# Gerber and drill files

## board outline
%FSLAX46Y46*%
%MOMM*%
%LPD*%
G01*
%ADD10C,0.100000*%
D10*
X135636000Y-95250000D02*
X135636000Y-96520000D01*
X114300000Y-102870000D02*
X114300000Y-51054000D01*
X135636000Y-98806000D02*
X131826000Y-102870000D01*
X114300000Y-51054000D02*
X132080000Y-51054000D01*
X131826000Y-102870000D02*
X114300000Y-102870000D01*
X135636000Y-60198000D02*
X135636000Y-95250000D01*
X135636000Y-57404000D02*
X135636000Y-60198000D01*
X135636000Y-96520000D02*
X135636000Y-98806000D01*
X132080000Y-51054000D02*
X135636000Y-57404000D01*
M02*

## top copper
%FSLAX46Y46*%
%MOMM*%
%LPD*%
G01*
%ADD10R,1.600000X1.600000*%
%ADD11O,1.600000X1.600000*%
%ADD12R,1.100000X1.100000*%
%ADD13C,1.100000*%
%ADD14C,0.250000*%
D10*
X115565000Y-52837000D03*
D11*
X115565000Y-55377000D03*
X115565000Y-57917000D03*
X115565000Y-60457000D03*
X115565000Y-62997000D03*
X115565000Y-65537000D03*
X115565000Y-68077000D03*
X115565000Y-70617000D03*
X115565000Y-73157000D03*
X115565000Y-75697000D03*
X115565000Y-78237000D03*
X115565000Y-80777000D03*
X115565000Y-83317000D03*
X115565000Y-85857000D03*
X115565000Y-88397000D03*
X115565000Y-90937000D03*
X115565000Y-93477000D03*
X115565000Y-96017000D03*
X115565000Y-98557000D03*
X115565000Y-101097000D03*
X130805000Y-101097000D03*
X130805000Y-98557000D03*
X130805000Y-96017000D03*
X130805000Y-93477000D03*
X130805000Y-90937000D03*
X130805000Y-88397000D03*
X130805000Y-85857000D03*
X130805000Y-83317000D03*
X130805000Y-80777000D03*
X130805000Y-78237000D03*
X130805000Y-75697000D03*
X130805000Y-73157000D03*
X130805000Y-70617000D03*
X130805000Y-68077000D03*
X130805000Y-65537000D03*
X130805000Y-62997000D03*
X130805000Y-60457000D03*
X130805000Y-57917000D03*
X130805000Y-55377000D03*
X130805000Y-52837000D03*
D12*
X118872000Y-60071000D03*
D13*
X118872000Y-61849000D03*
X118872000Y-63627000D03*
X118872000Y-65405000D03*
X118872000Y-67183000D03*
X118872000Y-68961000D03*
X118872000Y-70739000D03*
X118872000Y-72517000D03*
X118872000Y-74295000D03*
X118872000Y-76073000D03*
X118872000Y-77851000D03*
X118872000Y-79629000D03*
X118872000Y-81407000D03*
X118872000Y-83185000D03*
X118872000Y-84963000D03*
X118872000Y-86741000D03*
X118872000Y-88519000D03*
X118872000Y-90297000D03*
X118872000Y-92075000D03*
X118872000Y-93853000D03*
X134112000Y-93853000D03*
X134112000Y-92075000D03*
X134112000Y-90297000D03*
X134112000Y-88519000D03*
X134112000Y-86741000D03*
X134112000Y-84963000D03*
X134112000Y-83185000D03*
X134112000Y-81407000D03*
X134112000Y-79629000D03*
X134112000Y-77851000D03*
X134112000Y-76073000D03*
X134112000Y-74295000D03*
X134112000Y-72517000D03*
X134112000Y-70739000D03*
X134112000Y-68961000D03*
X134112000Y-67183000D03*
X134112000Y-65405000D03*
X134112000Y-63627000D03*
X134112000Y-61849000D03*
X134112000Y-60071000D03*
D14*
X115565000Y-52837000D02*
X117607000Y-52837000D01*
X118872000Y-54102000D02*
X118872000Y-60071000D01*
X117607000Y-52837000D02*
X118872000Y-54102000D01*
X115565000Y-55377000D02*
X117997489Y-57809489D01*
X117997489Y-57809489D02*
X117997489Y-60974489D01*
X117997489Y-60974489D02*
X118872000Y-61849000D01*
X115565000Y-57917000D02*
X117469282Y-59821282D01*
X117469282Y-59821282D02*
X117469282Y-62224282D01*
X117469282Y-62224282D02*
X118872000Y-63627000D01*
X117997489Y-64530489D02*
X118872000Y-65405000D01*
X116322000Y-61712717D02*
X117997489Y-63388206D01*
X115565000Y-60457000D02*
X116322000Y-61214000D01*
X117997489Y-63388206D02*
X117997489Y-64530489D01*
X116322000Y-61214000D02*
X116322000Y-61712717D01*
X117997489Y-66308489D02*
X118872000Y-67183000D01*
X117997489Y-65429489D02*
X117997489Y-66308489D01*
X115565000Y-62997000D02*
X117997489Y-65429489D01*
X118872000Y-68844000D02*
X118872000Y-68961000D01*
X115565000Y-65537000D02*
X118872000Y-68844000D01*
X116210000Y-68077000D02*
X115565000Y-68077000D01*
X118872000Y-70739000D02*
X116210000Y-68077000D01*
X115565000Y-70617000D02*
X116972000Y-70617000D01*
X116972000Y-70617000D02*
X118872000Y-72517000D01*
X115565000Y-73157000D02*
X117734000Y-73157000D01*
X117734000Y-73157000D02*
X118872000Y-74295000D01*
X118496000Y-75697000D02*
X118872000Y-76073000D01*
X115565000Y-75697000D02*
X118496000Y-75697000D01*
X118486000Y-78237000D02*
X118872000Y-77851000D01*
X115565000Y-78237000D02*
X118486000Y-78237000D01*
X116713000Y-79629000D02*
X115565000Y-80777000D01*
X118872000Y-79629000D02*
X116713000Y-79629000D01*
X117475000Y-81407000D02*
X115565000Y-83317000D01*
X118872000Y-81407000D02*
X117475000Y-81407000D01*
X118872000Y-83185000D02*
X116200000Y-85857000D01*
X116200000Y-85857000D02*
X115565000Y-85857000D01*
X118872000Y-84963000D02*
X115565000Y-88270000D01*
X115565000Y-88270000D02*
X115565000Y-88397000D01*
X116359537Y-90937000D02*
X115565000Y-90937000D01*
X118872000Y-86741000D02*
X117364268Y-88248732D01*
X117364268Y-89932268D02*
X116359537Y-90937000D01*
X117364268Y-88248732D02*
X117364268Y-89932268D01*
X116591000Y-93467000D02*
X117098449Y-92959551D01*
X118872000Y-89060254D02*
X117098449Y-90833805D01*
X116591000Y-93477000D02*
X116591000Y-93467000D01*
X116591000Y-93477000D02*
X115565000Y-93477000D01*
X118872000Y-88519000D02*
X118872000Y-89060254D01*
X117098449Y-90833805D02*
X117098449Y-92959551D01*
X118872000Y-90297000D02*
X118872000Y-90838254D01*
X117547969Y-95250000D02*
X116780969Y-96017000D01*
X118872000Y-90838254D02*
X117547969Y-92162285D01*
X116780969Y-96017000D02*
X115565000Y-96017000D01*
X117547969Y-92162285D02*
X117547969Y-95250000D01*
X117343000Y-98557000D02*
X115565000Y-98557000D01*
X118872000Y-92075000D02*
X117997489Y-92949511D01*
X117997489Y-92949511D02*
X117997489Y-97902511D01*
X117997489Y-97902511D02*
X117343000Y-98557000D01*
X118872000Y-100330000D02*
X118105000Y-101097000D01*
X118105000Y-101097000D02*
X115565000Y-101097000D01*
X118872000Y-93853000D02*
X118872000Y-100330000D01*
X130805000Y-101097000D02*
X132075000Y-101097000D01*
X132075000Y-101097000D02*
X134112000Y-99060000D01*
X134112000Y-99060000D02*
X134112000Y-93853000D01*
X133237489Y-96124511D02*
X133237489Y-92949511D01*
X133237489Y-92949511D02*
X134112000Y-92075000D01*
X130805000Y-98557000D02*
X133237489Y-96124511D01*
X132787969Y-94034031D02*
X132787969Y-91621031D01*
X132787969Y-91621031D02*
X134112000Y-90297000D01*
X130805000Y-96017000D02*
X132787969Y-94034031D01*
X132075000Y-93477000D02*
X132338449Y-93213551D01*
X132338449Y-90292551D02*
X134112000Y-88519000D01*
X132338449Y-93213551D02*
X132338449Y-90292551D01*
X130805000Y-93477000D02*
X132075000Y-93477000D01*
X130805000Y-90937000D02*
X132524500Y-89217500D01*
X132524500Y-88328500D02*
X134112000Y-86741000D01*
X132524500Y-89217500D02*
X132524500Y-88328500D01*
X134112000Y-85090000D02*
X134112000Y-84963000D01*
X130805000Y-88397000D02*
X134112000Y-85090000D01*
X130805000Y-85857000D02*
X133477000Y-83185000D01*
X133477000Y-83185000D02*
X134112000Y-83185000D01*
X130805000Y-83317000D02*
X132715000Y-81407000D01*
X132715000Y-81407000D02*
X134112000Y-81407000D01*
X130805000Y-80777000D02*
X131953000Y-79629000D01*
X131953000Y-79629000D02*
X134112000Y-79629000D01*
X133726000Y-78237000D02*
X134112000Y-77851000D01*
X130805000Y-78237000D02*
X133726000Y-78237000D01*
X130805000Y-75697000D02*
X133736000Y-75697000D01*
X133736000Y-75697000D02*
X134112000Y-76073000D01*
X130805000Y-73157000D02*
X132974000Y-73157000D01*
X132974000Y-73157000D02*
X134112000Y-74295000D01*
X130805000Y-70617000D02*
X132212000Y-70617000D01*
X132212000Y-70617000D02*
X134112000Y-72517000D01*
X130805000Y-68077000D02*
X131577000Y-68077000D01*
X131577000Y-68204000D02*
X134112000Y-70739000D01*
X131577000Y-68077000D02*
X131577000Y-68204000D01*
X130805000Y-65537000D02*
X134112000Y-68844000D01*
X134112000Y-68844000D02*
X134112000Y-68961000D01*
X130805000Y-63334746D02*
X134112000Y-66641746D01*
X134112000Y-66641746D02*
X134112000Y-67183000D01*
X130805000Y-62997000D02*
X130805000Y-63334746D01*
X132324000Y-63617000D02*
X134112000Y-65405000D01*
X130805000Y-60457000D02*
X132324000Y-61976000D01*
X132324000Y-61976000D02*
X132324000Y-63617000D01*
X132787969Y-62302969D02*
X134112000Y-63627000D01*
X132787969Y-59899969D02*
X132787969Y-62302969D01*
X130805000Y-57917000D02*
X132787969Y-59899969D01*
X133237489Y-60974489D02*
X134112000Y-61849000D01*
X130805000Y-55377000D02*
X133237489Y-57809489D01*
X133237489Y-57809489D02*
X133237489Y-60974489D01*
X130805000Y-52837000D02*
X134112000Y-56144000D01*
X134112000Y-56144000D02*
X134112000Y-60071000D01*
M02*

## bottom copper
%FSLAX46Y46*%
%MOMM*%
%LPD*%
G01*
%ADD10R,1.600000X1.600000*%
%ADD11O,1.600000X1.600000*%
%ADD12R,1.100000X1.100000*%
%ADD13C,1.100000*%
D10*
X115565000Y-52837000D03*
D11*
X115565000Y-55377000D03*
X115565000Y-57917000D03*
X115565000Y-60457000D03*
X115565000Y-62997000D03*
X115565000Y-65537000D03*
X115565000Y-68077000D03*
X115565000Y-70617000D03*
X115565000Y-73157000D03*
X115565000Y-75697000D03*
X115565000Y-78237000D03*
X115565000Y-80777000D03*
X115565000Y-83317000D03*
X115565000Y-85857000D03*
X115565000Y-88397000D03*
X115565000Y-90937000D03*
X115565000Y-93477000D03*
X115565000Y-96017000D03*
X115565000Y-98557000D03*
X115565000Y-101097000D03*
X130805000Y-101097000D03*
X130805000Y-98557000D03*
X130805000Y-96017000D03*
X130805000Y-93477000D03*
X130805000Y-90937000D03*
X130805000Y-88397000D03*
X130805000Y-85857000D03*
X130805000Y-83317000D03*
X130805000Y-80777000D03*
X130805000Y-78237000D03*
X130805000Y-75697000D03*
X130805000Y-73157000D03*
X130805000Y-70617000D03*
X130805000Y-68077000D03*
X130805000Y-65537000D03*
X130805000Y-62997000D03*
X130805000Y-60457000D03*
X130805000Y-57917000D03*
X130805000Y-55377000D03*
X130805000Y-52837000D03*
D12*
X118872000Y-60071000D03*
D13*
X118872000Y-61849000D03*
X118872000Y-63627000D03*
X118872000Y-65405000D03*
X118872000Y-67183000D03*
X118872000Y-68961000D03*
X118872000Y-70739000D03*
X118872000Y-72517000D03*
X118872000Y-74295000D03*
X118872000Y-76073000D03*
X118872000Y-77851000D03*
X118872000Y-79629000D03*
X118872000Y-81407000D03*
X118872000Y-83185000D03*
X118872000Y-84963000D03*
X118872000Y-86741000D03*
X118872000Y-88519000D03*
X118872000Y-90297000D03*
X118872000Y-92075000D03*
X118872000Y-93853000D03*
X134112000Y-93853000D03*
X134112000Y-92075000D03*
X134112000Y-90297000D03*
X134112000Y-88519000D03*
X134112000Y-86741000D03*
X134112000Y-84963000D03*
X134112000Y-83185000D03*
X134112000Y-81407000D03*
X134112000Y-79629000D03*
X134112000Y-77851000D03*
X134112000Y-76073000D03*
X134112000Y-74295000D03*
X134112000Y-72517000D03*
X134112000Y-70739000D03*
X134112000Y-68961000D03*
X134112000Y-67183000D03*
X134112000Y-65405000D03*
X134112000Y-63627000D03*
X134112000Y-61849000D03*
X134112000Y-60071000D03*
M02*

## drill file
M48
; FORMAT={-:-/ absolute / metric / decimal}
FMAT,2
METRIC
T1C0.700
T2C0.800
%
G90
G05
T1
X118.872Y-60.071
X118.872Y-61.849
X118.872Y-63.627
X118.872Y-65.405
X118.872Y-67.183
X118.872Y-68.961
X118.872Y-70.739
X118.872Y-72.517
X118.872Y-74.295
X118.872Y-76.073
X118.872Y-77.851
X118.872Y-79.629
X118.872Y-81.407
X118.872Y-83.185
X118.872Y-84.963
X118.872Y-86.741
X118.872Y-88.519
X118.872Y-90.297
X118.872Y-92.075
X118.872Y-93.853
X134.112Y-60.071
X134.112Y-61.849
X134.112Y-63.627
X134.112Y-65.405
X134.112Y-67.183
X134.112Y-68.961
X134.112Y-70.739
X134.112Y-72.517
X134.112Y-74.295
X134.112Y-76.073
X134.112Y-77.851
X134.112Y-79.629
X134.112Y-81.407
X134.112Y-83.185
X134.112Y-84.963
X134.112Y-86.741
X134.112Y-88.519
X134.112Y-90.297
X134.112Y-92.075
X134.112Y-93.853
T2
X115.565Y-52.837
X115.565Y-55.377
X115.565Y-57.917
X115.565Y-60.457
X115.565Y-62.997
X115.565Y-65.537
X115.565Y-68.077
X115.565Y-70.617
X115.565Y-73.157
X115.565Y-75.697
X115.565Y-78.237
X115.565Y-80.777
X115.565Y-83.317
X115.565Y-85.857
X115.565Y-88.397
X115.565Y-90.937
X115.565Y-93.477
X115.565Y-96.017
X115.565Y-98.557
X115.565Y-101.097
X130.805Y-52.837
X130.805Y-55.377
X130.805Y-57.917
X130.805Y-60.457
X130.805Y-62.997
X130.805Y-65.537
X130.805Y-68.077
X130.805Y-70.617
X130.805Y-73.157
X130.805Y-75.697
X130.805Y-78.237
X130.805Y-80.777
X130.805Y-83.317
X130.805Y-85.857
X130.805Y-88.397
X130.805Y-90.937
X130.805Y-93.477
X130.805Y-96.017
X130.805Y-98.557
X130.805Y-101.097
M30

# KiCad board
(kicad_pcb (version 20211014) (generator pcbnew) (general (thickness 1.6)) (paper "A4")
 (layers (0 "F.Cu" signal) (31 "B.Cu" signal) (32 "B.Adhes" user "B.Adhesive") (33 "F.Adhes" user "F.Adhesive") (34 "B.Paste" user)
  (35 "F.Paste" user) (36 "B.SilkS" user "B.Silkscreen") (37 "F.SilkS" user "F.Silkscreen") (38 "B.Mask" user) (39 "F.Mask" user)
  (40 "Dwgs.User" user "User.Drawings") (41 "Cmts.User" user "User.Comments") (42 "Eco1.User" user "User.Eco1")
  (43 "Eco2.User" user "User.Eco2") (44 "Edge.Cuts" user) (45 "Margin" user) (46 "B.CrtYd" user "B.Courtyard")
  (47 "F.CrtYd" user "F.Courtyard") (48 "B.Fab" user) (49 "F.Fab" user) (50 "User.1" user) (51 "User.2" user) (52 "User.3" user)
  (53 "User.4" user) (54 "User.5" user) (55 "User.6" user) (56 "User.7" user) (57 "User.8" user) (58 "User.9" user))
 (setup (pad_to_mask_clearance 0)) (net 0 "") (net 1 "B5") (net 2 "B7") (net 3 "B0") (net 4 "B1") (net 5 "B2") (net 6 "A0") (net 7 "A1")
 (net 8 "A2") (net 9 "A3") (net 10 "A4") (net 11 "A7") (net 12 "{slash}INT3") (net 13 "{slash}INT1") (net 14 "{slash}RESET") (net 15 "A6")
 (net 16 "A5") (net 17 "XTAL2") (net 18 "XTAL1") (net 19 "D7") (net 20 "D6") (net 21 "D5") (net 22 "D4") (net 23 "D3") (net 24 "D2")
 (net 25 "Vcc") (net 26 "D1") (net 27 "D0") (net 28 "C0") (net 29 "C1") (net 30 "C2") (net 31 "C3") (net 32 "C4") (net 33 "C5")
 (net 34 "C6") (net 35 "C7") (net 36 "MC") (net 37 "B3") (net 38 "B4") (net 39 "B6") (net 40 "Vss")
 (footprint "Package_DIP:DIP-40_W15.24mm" (layer "F.Cu") (at 115.565 52.837)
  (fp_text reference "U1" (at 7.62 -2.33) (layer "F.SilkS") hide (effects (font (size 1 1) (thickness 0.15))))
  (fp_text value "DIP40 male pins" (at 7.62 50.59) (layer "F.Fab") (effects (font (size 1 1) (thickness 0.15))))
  (pad "1" thru_hole rect locked (at 0 0) (size 1.6 1.6) (drill 0.8) (layers *.Cu *.Mask) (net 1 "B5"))
  (pad "2" thru_hole oval locked (at 0 2.54) (size 1.6 1.6) (drill 0.8) (layers *.Cu *.Mask) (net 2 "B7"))
  (pad "3" thru_hole oval locked (at 0 5.08) (size 1.6 1.6) (drill 0.8) (layers *.Cu *.Mask) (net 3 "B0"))
  (pad "4" thru_hole oval locked (at 0 7.62) (size 1.6 1.6) (drill 0.8) (layers *.Cu *.Mask) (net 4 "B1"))
  (pad "5" thru_hole oval locked (at 0 10.16) (size 1.6 1.6) (drill 0.8) (layers *.Cu *.Mask) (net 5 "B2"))
  (pad "6" thru_hole oval locked (at 0 12.7) (size 1.6 1.6) (drill 0.8) (layers *.Cu *.Mask) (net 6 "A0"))
  (pad "7" thru_hole oval locked (at 0 15.24) (size 1.6 1.6) (drill 0.8) (layers *.Cu *.Mask) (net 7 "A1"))
  (pad "8" thru_hole oval locked (at 0 17.78) (size 1.6 1.6) (drill 0.8) (layers *.Cu *.Mask) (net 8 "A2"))
  (pad "9" thru_hole oval locked (at 0 20.32) (size 1.6 1.6) (drill 0.8) (layers *.Cu *.Mask) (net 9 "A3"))
  (pad "10" thru_hole oval locked (at 0 22.86) (size 1.6 1.6) (drill 0.8) (layers *.Cu *.Mask) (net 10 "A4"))
  (pad "11" thru_hole oval locked (at 0 25.4) (size 1.6 1.6) (drill 0.8) (layers *.Cu *.Mask) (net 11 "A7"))
  (pad "12" thru_hole oval locked (at 0 27.94) (size 1.6 1.6) (drill 0.8) (layers *.Cu *.Mask) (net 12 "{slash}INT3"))
  (pad "13" thru_hole oval locked (at 0 30.48) (size 1.6 1.6) (drill 0.8) (layers *.Cu *.Mask) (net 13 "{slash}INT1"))
  (pad "14" thru_hole oval locked (at 0 33.02) (size 1.6 1.6) (drill 0.8) (layers *.Cu *.Mask) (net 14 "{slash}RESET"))
  (pad "15" thru_hole oval locked (at 0 35.56) (size 1.6 1.6) (drill 0.8) (layers *.Cu *.Mask) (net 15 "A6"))
  (pad "16" thru_hole oval locked (at 0 38.1) (size 1.6 1.6) (drill 0.8) (layers *.Cu *.Mask) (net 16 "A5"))
  (pad "17" thru_hole oval locked (at 0 40.64) (size 1.6 1.6) (drill 0.8) (layers *.Cu *.Mask) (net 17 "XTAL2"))
  (pad "18" thru_hole oval locked (at 0 43.18) (size 1.6 1.6) (drill 0.8) (layers *.Cu *.Mask) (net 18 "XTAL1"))
  (pad "19" thru_hole oval locked (at 0 45.72) (size 1.6 1.6) (drill 0.8) (layers *.Cu *.Mask) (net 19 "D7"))
  (pad "20" thru_hole oval locked (at 0 48.26) (size 1.6 1.6) (drill 0.8) (layers *.Cu *.Mask) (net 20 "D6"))
  (pad "21" thru_hole oval locked (at 15.24 48.26) (size 1.6 1.6) (drill 0.8) (layers *.Cu *.Mask) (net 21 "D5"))
  (pad "22" thru_hole oval locked (at 15.24 45.72) (size 1.6 1.6) (drill 0.8) (layers *.Cu *.Mask) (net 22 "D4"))
  (pad "23" thru_hole oval locked (at 15.24 43.18) (size 1.6 1.6) (drill 0.8) (layers *.Cu *.Mask) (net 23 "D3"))
  (pad "24" thru_hole oval locked (at 15.24 40.64) (size 1.6 1.6) (drill 0.8) (layers *.Cu *.Mask) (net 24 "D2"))
  (pad "25" thru_hole oval locked (at 15.24 38.1) (size 1.6 1.6) (drill 0.8) (layers *.Cu *.Mask) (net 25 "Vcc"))
  (pad "26" thru_hole oval locked (at 15.24 35.56) (size 1.6 1.6) (drill 0.8) (layers *.Cu *.Mask) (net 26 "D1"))
  (pad "27" thru_hole oval locked (at 15.24 33.02) (size 1.6 1.6) (drill 0.8) (layers *.Cu *.Mask) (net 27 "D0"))
  (pad "28" thru_hole oval locked (at 15.24 30.48) (size 1.6 1.6) (drill 0.8) (layers *.Cu *.Mask) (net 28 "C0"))
  (pad "29" thru_hole oval locked (at 15.24 27.94) (size 1.6 1.6) (drill 0.8) (layers *.Cu *.Mask) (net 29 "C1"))
  (pad "30" thru_hole oval locked (at 15.24 25.4) (size 1.6 1.6) (drill 0.8) (layers *.Cu *.Mask) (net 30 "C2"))
  (pad "31" thru_hole oval locked (at 15.24 22.86) (size 1.6 1.6) (drill 0.8) (layers *.Cu *.Mask) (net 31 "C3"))
  (pad "32" thru_hole oval locked (at 15.24 20.32) (size 1.6 1.6) (drill 0.8) (layers *.Cu *.Mask) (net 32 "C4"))
  (pad "33" thru_hole oval locked (at 15.24 17.78) (size 1.6 1.6) (drill 0.8) (layers *.Cu *.Mask) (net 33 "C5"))
  (pad "34" thru_hole oval locked (at 15.24 15.24) (size 1.6 1.6) (drill 0.8) (layers *.Cu *.Mask) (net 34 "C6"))
  (pad "35" thru_hole oval locked (at 15.24 12.7) (size 1.6 1.6) (drill 0.8) (layers *.Cu *.Mask) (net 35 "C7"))
  (pad "36" thru_hole oval locked (at 15.24 10.16) (size 1.6 1.6) (drill 0.8) (layers *.Cu *.Mask) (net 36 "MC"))
  (pad "37" thru_hole oval locked (at 15.24 7.62) (size 1.6 1.6) (drill 0.8) (layers *.Cu *.Mask) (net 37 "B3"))
  (pad "38" thru_hole oval locked (at 15.24 5.08) (size 1.6 1.6) (drill 0.8) (layers *.Cu *.Mask) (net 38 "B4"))
  (pad "39" thru_hole oval locked (at 15.24 2.54) (size 1.6 1.6) (drill 0.8) (layers *.Cu *.Mask) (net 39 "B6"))
  (pad "40" thru_hole oval locked (at 15.24 0) (size 1.6 1.6) (drill 0.8) (layers *.Cu *.Mask) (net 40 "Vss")))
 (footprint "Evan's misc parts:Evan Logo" (layer "F.Cu") (at 123.444 99.568)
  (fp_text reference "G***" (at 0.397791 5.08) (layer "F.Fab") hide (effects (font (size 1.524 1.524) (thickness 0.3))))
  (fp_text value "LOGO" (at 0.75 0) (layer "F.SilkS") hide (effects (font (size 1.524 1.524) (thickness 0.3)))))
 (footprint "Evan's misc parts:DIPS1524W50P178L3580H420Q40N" (layer "F.Cu") (at 118.872 60.071)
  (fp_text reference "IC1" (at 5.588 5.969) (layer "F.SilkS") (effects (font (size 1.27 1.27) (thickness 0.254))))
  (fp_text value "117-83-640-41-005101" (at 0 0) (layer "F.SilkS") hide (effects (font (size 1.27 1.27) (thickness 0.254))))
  (pad "1" thru_hole rect (at 0 0) (size 1.1 1.1) (drill 0.7) (layers *.Cu *.Mask) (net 1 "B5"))
  (pad "2" thru_hole circle (at 0 1.778) (size 1.1 1.1) (drill 0.7) (layers *.Cu *.Mask) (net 2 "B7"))
  (pad "3" thru_hole circle (at 0 3.556) (size 1.1 1.1) (drill 0.7) (layers *.Cu *.Mask) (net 3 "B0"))
  (pad "4" thru_hole circle (at 0 5.334) (size 1.1 1.1) (drill 0.7) (layers *.Cu *.Mask) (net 4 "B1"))
  (pad "5" thru_hole circle (at 0 7.112) (size 1.1 1.1) (drill 0.7) (layers *.Cu *.Mask) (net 5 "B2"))
  (pad "6" thru_hole circle (at 0 8.89) (size 1.1 1.1) (drill 0.7) (layers *.Cu *.Mask) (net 6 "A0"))
  (pad "7" thru_hole circle (at 0 10.668) (size 1.1 1.1) (drill 0.7) (layers *.Cu *.Mask) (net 7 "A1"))
  (pad "8" thru_hole circle (at 0 12.446) (size 1.1 1.1) (drill 0.7) (layers *.Cu *.Mask) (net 8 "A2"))
  (pad "9" thru_hole circle (at 0 14.224) (size 1.1 1.1) (drill 0.7) (layers *.Cu *.Mask) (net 9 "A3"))
  (pad "10" thru_hole circle (at 0 16.002) (size 1.1 1.1) (drill 0.7) (layers *.Cu *.Mask) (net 10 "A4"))
  (pad "11" thru_hole circle (at 0 17.78) (size 1.1 1.1) (drill 0.7) (layers *.Cu *.Mask) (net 11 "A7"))
  (pad "12" thru_hole circle (at 0 19.558) (size 1.1 1.1) (drill 0.7) (layers *.Cu *.Mask) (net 12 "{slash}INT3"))
  (pad "13" thru_hole circle (at 0 21.336) (size 1.1 1.1) (drill 0.7) (layers *.Cu *.Mask) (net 13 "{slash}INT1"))
  (pad "14" thru_hole circle (at 0 23.114) (size 1.1 1.1) (drill 0.7) (layers *.Cu *.Mask) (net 14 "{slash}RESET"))
  (pad "15" thru_hole circle (at 0 24.892) (size 1.1 1.1) (drill 0.7) (layers *.Cu *.Mask) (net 15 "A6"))
  (pad "16" thru_hole circle (at 0 26.67) (size 1.1 1.1) (drill 0.7) (layers *.Cu *.Mask) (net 16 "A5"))
  (pad "17" thru_hole circle (at 0 28.448) (size 1.1 1.1) (drill 0.7) (layers *.Cu *.Mask) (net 17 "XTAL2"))
  (pad "18" thru_hole circle (at 0 30.226) (size 1.1 1.1) (drill 0.7) (layers *.Cu *.Mask) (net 18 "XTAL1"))
  (pad "19" thru_hole circle (at 0 32.004) (size 1.1 1.1) (drill 0.7) (layers *.Cu *.Mask) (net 19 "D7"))
  (pad "20" thru_hole circle (at 0 33.782) (size 1.1 1.1) (drill 0.7) (layers *.Cu *.Mask) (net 20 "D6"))
  (pad "21" thru_hole circle (at 15.24 33.782) (size 1.1 1.1) (drill 0.7) (layers *.Cu *.Mask) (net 21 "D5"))
  (pad "22" thru_hole circle (at 15.24 32.004) (size 1.1 1.1) (drill 0.7) (layers *.Cu *.Mask) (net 22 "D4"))
  (pad "23" thru_hole circle (at 15.24 30.226) (size 1.1 1.1) (drill 0.7) (layers *.Cu *.Mask) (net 23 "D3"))
  (pad "24" thru_hole circle (at 15.24 28.448) (size 1.1 1.1) (drill 0.7) (layers *.Cu *.Mask) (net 24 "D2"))
  (pad "25" thru_hole circle (at 15.24 26.67) (size 1.1 1.1) (drill 0.7) (layers *.Cu *.Mask) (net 25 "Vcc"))
  (pad "26" thru_hole circle (at 15.24 24.892) (size 1.1 1.1) (drill 0.7) (layers *.Cu *.Mask) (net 26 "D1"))
  (pad "27" thru_hole circle (at 15.24 23.114) (size 1.1 1.1) (drill 0.7) (layers *.Cu *.Mask) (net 27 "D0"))
  (pad "28" thru_hole circle (at 15.24 21.336) (size 1.1 1.1) (drill 0.7) (layers *.Cu *.Mask) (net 28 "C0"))
  (pad "29" thru_hole circle (at 15.24 19.558) (size 1.1 1.1) (drill 0.7) (layers *.Cu *.Mask) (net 29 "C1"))
  (pad "30" thru_hole circle (at 15.24 17.78) (size 1.1 1.1) (drill 0.7) (layers *.Cu *.Mask) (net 30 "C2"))
  (pad "31" thru_hole circle (at 15.24 16.002) (size 1.1 1.1) (drill 0.7) (layers *.Cu *.Mask) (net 31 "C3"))
  (pad "32" thru_hole circle (at 15.24 14.224) (size 1.1 1.1) (drill 0.7) (layers *.Cu *.Mask) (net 32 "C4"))
  (pad "33" thru_hole circle (at 15.24 12.446) (size 1.1 1.1) (drill 0.7) (layers *.Cu *.Mask) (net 33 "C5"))
  (pad "34" thru_hole circle (at 15.24 10.668) (size 1.1 1.1) (drill 0.7) (layers *.Cu *.Mask) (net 34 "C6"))
  (pad "35" thru_hole circle (at 15.24 8.89) (size 1.1 1.1) (drill 0.7) (layers *.Cu *.Mask) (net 35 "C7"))
  (pad "36" thru_hole circle (at 15.24 7.112) (size 1.1 1.1) (drill 0.7) (layers *.Cu *.Mask) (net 36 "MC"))
  (pad "37" thru_hole circle (at 15.24 5.334) (size 1.1 1.1) (drill 0.7) (layers *.Cu *.Mask) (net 37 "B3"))
  (pad "38" thru_hole circle (at 15.24 3.556) (size 1.1 1.1) (drill 0.7) (layers *.Cu *.Mask) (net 38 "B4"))
  (pad "39" thru_hole circle (at 15.24 1.778) (size 1.1 1.1) (drill 0.7) (layers *.Cu *.Mask) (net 39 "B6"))
  (pad "40" thru_hole circle (at 15.24 0) (size 1.1 1.1) (drill 0.7) (layers *.Cu *.Mask) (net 40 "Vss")))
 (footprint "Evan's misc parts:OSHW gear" (layer "B.Cu") (at 123.444 98.552 180)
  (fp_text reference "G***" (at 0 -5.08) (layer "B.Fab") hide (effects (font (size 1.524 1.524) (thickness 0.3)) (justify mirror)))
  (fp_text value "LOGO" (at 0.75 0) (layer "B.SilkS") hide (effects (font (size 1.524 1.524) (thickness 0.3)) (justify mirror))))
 (gr_line (start 135.636 95.25) (end 135.636 96.52) (layer "Edge.Cuts") (width 0.1))
 (gr_line (start 114.3 102.87) (end 114.3 51.054) (layer "Edge.Cuts") (width 0.1))
 (gr_line (start 135.636 98.806) (end 131.826 102.87) (layer "Edge.Cuts") (width 0.1))
 (gr_line (start 114.3 51.054) (end 132.08 51.054) (layer "Edge.Cuts") (width 0.1))
 (gr_line (start 131.826 102.87) (end 114.3 102.87) (layer "Edge.Cuts") (width 0.1))
 (gr_line (start 135.636 60.198) (end 135.636 95.25) (layer "Edge.Cuts") (width 0.1))
 (gr_line (start 135.636 57.404) (end 135.636 60.198) (layer "Edge.Cuts") (width 0.1))
 (gr_line (start 135.636 96.52) (end 135.636 98.806) (layer "Edge.Cuts") (width 0.1))
 (gr_line (start 132.08 51.054) (end 135.636 57.404) (layer "Edge.Cuts") (width 0.1))
 (segment (start 115.565 52.837) (end 117.607 52.837) (width 0.25) (layer "F.Cu") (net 1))
 (segment (start 118.872 54.102) (end 118.872 60.071) (width 0.25) (layer "F.Cu") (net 1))
 (segment (start 117.607 52.837) (end 118.872 54.102) (width 0.25) (layer "F.Cu") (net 1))
 (segment (start 115.565 55.377) (end 117.997489 57.809489) (width 0.25) (layer "F.Cu") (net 2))
 (segment (start 117.997489 57.809489) (end 117.997489 60.974489) (width 0.25) (layer "F.Cu") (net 2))
 (segment (start 117.997489 60.974489) (end 118.872 61.849) (width 0.25) (layer "F.Cu") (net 2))
 (segment (start 115.565 57.917) (end 117.469282 59.821282) (width 0.25) (layer "F.Cu") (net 3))
 (segment (start 117.469282 59.821282) (end 117.469282 62.224282) (width 0.25) (layer "F.Cu") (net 3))
 (segment (start 117.469282 62.224282) (end 118.872 63.627) (width 0.25) (layer "F.Cu") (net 3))
 (segment (start 117.997489 64.530489) (end 118.872 65.405) (width 0.25) (layer "F.Cu") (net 4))
 (segment (start 116.322 61.712717) (end 117.997489 63.388206) (width 0.25) (layer "F.Cu") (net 4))
 (segment (start 115.565 60.457) (end 116.322 61.214) (width 0.25) (layer "F.Cu") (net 4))
 (segment (start 117.997489 63.388206) (end 117.997489 64.530489) (width 0.25) (layer "F.Cu") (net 4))
 (segment (start 116.322 61.214) (end 116.322 61.712717) (width 0.25) (layer "F.Cu") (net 4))
 (segment (start 117.997489 66.308489) (end 118.872 67.183) (width 0.25) (layer "F.Cu") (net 5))
 (segment (start 117.997489 65.429489) (end 117.997489 66.308489) (width 0.25) (layer "F.Cu") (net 5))
 (segment (start 115.565 62.997) (end 117.997489 65.429489) (width 0.25) (layer "F.Cu") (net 5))
 (segment (start 118.872 68.844) (end 118.872 68.961) (width 0.25) (layer "F.Cu") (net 6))
 (segment (start 115.565 65.537) (end 118.872 68.844) (width 0.25) (layer "F.Cu") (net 6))
 (segment (start 116.21 68.077) (end 115.565 68.077) (width 0.25) (layer "F.Cu") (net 7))
 (segment (start 118.872 70.739) (end 116.21 68.077) (width 0.25) (layer "F.Cu") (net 7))
 (segment (start 115.565 70.617) (end 116.972 70.617) (width 0.25) (layer "F.Cu") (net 8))
 (segment (start 116.972 70.617) (end 118.872 72.517) (width 0.25) (layer "F.Cu") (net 8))
 (segment (start 115.565 73.157) (end 117.734 73.157) (width 0.25) (layer "F.Cu") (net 9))
 (segment (start 117.734 73.157) (end 118.872 74.295) (width 0.25) (layer "F.Cu") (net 9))
 (segment (start 118.496 75.697) (end 118.872 76.073) (width 0.25) (layer "F.Cu") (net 10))
 (segment (start 115.565 75.697) (end 118.496 75.697) (width 0.25) (layer "F.Cu") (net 10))
 (segment (start 118.486 78.237) (end 118.872 77.851) (width 0.25) (layer "F.Cu") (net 11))
 (segment (start 115.565 78.237) (end 118.486 78.237) (width 0.25) (layer "F.Cu") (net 11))
 (segment (start 116.713 79.629) (end 115.565 80.777) (width 0.25) (layer "F.Cu") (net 12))
 (segment (start 118.872 79.629) (end 116.713 79.629) (width 0.25) (layer "F.Cu") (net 12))
 (segment (start 117.475 81.407) (end 115.565 83.317) (width 0.25) (layer "F.Cu") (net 13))
 (segment (start 118.872 81.407) (end 117.475 81.407) (width 0.25) (layer "F.Cu") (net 13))
 (segment (start 118.872 83.185) (end 116.2 85.857) (width 0.25) (layer "F.Cu") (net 14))
 (segment (start 116.2 85.857) (end 115.565 85.857) (width 0.25) (layer "F.Cu") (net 14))
 (segment (start 118.872 84.963) (end 115.565 88.27) (width 0.25) (layer "F.Cu") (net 15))
 (segment (start 115.565 88.27) (end 115.565 88.397) (width 0.25) (layer "F.Cu") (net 15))
 (segment (start 116.359537 90.937) (end 115.565 90.937) (width 0.25) (layer "F.Cu") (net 16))
 (segment (start 118.872 86.741) (end 117.364268 88.248732) (width 0.25) (layer "F.Cu") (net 16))
 (segment (start 117.364268 89.932268) (end 116.359537 90.937) (width 0.25) (layer "F.Cu") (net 16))
 (segment (start 117.364268 88.248732) (end 117.364268 89.932268) (width 0.25) (layer "F.Cu") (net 16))
 (segment (start 116.591 93.467) (end 117.098449 92.959551) (width 0.25) (layer "F.Cu") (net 17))
 (segment (start 118.872 89.060254) (end 117.098449 90.833805) (width 0.25) (layer "F.Cu") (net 17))
 (segment (start 116.591 93.477) (end 116.591 93.467) (width 0.25) (layer "F.Cu") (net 17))
 (segment (start 116.591 93.477) (end 115.565 93.477) (width 0.25) (layer "F.Cu") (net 17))
 (segment (start 118.872 88.519) (end 118.872 89.060254) (width 0.25) (layer "F.Cu") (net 17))
 (segment (start 117.098449 90.833805) (end 117.098449 92.959551) (width 0.25) (layer "F.Cu") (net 17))
 (segment (start 118.872 90.297) (end 118.872 90.838254) (width 0.25) (layer "F.Cu") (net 18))
 (segment (start 117.547969 95.25) (end 116.780969 96.017) (width 0.25) (layer "F.Cu") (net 18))
 (segment (start 118.872 90.838254) (end 117.547969 92.162285) (width 0.25) (layer "F.Cu") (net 18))
 (segment (start 116.780969 96.017) (end 115.565 96.017) (width 0.25) (layer "F.Cu") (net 18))
 (segment (start 117.547969 92.162285) (end 117.547969 95.25) (width 0.25) (layer "F.Cu") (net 18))
 (segment (start 117.343 98.557) (end 115.565 98.557) (width 0.25) (layer "F.Cu") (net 19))
 (segment (start 118.872 92.075) (end 117.997489 92.949511) (width 0.25) (layer "F.Cu") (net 19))
 (segment (start 117.997489 92.949511) (end 117.997489 97.902511) (width 0.25) (layer "F.Cu") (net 19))
 (segment (start 117.997489 97.902511) (end 117.343 98.557) (width 0.25) (layer "F.Cu") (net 19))
 (segment (start 118.872 100.33) (end 118.105 101.097) (width 0.25) (layer "F.Cu") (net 20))
 (segment (start 118.105 101.097) (end 115.565 101.097) (width 0.25) (layer "F.Cu") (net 20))
 (segment (start 118.872 93.853) (end 118.872 100.33) (width 0.25) (layer "F.Cu") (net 20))
 (segment (start 130.805 101.097) (end 132.075 101.097) (width 0.25) (layer "F.Cu") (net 21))
 (segment (start 132.075 101.097) (end 134.112 99.06) (width 0.25) (layer "F.Cu") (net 21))
 (segment (start 134.112 99.06) (end 134.112 93.853) (width 0.25) (layer "F.Cu") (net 21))
 (segment (start 133.237489 96.124511) (end 133.237489 92.949511) (width 0.25) (layer "F.Cu") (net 22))
 (segment (start 133.237489 92.949511) (end 134.112 92.075) (width 0.25) (layer "F.Cu") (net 22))
 (segment (start 130.805 98.557) (end 133.237489 96.124511) (width 0.25) (layer "F.Cu") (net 22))
 (segment (start 132.787969 94.034031) (end 132.787969 91.621031) (width 0.25) (layer "F.Cu") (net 23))
 (segment (start 132.787969 91.621031) (end 134.112 90.297) (width 0.25) (layer "F.Cu") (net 23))
 (segment (start 130.805 96.017) (end 132.787969 94.034031) (width 0.25) (layer "F.Cu") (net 23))
 (segment (start 132.075 93.477) (end 132.338449 93.213551) (width 0.25) (layer "F.Cu") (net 24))
 (segment (start 132.338449 90.292551) (end 134.112 88.519) (width 0.25) (layer "F.Cu") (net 24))
 (segment (start 132.338449 93.213551) (end 132.338449 90.292551) (width 0.25) (layer "F.Cu") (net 24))
 (segment (start 130.805 93.477) (end 132.075 93.477) (width 0.25) (layer "F.Cu") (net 24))
 (segment (start 130.805 90.937) (end 132.5245 89.2175) (width 0.25) (layer "F.Cu") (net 25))
 (segment (start 132.5245 88.3285) (end 134.112 86.741) (width 0.25) (layer "F.Cu") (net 25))
 (segment (start 132.5245 89.2175) (end 132.5245 88.3285) (width 0.25) (layer "F.Cu") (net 25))
 (segment (start 134.112 85.09) (end 134.112 84.963) (width 0.25) (layer "F.Cu") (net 26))
 (segment (start 130.805 88.397) (end 134.112 85.09) (width 0.25) (layer "F.Cu") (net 26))
 (segment (start 130.805 85.857) (end 133.477 83.185) (width 0.25) (layer "F.Cu") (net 27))
 (segment (start 133.477 83.185) (end 134.112 83.185) (width 0.25) (layer "F.Cu") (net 27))
 (segment (start 130.805 83.317) (end 132.715 81.407) (width 0.25) (layer "F.Cu") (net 28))
 (segment (start 132.715 81.407) (end 134.112 81.407) (width 0.25) (layer "F.Cu") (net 28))
 (segment (start 130.805 80.777) (end 131.953 79.629) (width 0.25) (layer "F.Cu") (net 29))
 (segment (start 131.953 79.629) (end 134.112 79.629) (width 0.25) (layer "F.Cu") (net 29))
 (segment (start 133.726 78.237) (end 134.112 77.851) (width 0.25) (layer "F.Cu") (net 30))
 (segment (start 130.805 78.237) (end 133.726 78.237) (width 0.25) (layer "F.Cu") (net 30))
 (segment (start 130.805 75.697) (end 133.736 75.697) (width 0.25) (layer "F.Cu") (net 31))
 (segment (start 133.736 75.697) (end 134.112 76.073) (width 0.25) (layer "F.Cu") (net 31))
 (segment (start 130.805 73.157) (end 132.974 73.157) (width 0.25) (layer "F.Cu") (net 32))
 (segment (start 132.974 73.157) (end 134.112 74.295) (width 0.25) (layer "F.Cu") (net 32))
 (segment (start 130.805 70.617) (end 132.212 70.617) (width 0.25) (layer "F.Cu") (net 33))
 (segment (start 132.212 70.617) (end 134.112 72.517) (width 0.25) (layer "F.Cu") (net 33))
 (segment (start 130.805 68.077) (end 131.577 68.077) (width 0.25) (layer "F.Cu") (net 34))
 (segment (start 131.577 68.204) (end 134.112 70.739) (width 0.25) (layer "F.Cu") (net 34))
 (segment (start 131.577 68.077) (end 131.577 68.204) (width 0.25) (layer "F.Cu") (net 34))
 (segment (start 130.805 65.537) (end 134.112 68.844) (width 0.25) (layer "F.Cu") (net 35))
 (segment (start 134.112 68.844) (end 134.112 68.961) (width 0.25) (layer "F.Cu") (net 35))
 (segment (start 130.805 63.334746) (end 134.112 66.641746) (width 0.25) (layer "F.Cu") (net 36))
 (segment (start 134.112 66.641746) (end 134.112 67.183) (width 0.25) (layer "F.Cu") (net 36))
 (segment (start 130.805 62.997) (end 130.805 63.334746) (width 0.25) (layer "F.Cu") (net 36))
 (segment (start 132.324 63.617) (end 134.112 65.405) (width 0.25) (layer "F.Cu") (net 37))
 (segment (start 130.805 60.457) (end 132.324 61.976) (width 0.25) (layer "F.Cu") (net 37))
 (segment (start 132.324 61.976) (end 132.324 63.617) (width 0.25) (layer "F.Cu") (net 37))
 (segment (start 132.787969 62.302969) (end 134.112 63.627) (width 0.25) (layer "F.Cu") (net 38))
 (segment (start 132.787969 59.899969) (end 132.787969 62.302969) (width 0.25) (layer "F.Cu") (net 38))
 (segment (start 130.805 57.917) (end 132.787969 59.899969) (width 0.25) (layer "F.Cu") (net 38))
 (segment (start 133.237489 60.974489) (end 134.112 61.849) (width 0.25) (layer "F.Cu") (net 39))
 (segment (start 130.805 55.377) (end 133.237489 57.809489) (width 0.25) (layer "F.Cu") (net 39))
 (segment (start 133.237489 57.809489) (end 133.237489 60.974489) (width 0.25) (layer "F.Cu") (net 39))
 (segment (start 130.805 52.837) (end 134.112 56.144) (width 0.25) (layer "F.Cu") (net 40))
 (segment (start 134.112 56.144) (end 134.112 60.071) (width 0.25) (layer "F.Cu") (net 40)))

